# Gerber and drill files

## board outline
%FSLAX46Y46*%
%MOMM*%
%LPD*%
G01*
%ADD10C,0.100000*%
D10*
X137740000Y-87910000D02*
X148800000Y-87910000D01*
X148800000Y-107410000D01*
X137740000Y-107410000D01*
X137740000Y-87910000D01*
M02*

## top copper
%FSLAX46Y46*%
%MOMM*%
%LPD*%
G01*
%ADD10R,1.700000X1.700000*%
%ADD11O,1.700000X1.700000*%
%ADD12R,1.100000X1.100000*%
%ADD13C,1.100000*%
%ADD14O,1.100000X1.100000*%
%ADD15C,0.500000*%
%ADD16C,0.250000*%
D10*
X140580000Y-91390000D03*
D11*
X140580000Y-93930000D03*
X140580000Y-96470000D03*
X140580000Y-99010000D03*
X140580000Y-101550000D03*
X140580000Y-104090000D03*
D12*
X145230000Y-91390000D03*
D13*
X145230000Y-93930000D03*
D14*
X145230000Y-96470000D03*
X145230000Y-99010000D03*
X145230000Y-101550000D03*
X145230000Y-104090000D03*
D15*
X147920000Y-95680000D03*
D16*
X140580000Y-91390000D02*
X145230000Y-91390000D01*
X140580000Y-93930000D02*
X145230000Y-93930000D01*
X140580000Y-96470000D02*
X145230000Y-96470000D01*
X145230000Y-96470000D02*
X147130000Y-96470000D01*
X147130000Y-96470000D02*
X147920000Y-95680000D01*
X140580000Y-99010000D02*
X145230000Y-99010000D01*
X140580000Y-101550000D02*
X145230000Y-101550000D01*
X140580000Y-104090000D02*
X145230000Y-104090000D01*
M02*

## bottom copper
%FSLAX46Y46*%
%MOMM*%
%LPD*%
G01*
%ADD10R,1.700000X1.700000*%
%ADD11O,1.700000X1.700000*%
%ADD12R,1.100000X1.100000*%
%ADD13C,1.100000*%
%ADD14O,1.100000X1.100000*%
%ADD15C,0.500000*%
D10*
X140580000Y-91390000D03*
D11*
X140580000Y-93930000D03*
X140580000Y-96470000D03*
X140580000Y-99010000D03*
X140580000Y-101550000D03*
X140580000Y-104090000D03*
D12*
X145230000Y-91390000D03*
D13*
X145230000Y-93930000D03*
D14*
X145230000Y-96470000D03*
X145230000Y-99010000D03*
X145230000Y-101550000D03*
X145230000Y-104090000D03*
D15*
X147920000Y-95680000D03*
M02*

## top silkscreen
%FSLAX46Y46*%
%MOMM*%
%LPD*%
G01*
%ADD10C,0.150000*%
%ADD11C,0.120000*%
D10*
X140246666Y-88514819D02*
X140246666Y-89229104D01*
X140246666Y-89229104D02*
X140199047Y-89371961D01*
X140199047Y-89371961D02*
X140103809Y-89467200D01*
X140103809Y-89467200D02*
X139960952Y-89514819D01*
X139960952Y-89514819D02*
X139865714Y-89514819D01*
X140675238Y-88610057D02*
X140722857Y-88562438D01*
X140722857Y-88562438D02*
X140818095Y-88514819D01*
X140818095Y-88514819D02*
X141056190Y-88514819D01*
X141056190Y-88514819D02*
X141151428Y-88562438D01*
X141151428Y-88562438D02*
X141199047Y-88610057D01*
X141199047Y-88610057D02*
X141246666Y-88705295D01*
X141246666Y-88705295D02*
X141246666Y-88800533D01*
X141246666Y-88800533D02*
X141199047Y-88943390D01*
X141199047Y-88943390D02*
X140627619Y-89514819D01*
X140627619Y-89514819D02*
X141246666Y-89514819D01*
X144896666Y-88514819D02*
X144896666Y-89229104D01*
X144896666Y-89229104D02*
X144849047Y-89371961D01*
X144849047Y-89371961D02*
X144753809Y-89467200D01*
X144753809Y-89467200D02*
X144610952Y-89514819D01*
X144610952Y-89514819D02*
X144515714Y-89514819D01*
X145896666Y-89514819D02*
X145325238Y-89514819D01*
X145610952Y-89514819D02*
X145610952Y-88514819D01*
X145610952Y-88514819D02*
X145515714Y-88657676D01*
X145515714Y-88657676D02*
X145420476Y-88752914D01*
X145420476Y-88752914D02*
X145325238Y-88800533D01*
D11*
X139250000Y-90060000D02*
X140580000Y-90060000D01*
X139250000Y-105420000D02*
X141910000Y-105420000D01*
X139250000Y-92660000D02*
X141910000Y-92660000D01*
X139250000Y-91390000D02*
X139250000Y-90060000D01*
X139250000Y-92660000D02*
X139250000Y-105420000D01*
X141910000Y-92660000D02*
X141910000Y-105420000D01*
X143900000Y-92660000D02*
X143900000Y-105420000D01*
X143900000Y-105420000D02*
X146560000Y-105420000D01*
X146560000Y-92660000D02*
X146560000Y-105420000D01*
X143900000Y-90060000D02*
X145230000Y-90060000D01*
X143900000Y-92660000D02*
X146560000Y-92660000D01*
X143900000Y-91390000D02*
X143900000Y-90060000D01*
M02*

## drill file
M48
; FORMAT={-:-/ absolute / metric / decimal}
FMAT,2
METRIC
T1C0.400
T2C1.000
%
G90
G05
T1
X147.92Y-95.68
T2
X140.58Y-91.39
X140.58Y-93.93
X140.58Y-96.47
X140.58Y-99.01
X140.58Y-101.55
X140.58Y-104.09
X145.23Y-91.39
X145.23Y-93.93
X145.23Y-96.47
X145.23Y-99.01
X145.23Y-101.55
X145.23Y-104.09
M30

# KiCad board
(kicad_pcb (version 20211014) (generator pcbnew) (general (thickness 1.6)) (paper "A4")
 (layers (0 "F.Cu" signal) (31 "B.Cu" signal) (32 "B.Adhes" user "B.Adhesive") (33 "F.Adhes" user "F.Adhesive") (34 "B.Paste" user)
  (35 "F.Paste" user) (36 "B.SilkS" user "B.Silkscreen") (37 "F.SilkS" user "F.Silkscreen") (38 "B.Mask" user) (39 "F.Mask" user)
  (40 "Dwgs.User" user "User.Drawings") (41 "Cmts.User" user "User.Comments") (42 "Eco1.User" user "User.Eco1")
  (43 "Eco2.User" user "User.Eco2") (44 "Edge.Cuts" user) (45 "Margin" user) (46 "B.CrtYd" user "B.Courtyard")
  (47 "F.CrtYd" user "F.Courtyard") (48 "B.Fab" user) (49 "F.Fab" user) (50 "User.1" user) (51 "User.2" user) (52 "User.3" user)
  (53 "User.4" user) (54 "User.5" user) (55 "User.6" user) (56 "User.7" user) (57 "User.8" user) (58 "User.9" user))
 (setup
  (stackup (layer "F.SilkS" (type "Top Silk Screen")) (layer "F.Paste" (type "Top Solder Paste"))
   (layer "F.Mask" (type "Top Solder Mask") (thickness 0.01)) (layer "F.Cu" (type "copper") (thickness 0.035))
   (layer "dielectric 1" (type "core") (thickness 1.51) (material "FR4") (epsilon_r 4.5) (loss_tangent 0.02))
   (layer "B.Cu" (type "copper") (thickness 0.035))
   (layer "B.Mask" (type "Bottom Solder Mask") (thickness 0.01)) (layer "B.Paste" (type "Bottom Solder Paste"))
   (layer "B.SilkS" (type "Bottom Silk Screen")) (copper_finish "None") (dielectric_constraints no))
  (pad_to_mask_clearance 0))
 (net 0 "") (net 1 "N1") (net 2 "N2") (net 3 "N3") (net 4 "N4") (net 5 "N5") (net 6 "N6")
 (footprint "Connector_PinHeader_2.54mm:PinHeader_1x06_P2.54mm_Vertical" (layer "F.Cu") (at 140.58 91.39)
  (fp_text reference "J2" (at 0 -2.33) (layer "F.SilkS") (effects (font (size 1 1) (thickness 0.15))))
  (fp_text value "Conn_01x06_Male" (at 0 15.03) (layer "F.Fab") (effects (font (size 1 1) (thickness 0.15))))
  (fp_line (start -1.33 -1.33) (end 0 -1.33) (layer "F.SilkS") (width 0.12))
  (fp_line (start -1.33 14.03) (end 1.33 14.03) (layer "F.SilkS") (width 0.12))
  (fp_line (start -1.33 1.27) (end 1.33 1.27) (layer "F.SilkS") (width 0.12))
  (fp_line (start -1.33 0) (end -1.33 -1.33) (layer "F.SilkS") (width 0.12))
  (fp_line (start -1.33 1.27) (end -1.33 14.03) (layer "F.SilkS") (width 0.12))
  (fp_line (start 1.33 1.27) (end 1.33 14.03) (layer "F.SilkS") (width 0.12))
  (pad "1" thru_hole rect (at 0 0) (size 1.7 1.7) (drill 1) (layers *.Cu *.Mask) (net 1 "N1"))
  (pad "2" thru_hole oval (at 0 2.54) (size 1.7 1.7) (drill 1) (layers *.Cu *.Mask) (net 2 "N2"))
  (pad "3" thru_hole oval (at 0 5.08) (size 1.7 1.7) (drill 1) (layers *.Cu *.Mask) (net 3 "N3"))
  (pad "4" thru_hole oval (at 0 7.62) (size 1.7 1.7) (drill 1) (layers *.Cu *.Mask) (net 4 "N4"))
  (pad "5" thru_hole oval (at 0 10.16) (size 1.7 1.7) (drill 1) (layers *.Cu *.Mask) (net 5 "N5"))
  (pad "6" thru_hole oval (at 0 12.7) (size 1.7 1.7) (drill 1) (layers *.Cu *.Mask) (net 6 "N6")))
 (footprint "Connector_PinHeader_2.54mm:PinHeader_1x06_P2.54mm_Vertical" (layer "F.Cu") (at 145.23 91.39)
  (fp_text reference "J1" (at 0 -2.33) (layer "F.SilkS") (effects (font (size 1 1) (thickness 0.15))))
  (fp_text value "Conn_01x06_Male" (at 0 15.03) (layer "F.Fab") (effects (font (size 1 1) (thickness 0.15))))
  (fp_line (start -1.33 1.27) (end -1.33 14.03) (layer "F.SilkS") (width 0.12))
  (fp_line (start -1.33 14.03) (end 1.33 14.03) (layer "F.SilkS") (width 0.12))
  (fp_line (start 1.33 1.27) (end 1.33 14.03) (layer "F.SilkS") (width 0.12))
  (fp_line (start -1.33 -1.33) (end 0 -1.33) (layer "F.SilkS") (width 0.12))
  (fp_line (start -1.33 1.27) (end 1.33 1.27) (layer "F.SilkS") (width 0.12))
  (fp_line (start -1.33 0) (end -1.33 -1.33) (layer "F.SilkS") (width 0.12))
  (pad "1" thru_hole rect (at 0 0) (size 1.1 1.1) (drill 1) (layers *.Cu *.Mask) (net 1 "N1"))
  (pad "2" thru_hole circle (at 0 2.54) (size 1.1 1.1) (drill 1) (layers *.Cu *.Mask) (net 2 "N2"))
  (pad "3" thru_hole oval (at 0 5.08) (size 1.1 1.1) (drill 1) (layers *.Cu *.Mask) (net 3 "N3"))
  (pad "4" thru_hole oval (at 0 7.62) (size 1.1 1.1) (drill 1) (layers *.Cu *.Mask) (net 4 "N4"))
  (pad "5" thru_hole oval (at 0 10.16) (size 1.1 1.1) (drill 1) (layers *.Cu *.Mask) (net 5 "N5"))
  (pad "6" thru_hole oval (at 0 12.7) (size 1.1 1.1) (drill 1) (layers *.Cu *.Mask) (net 6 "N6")))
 (gr_rect (start 137.74 87.91) (end 148.8 107.41) (layer "Edge.Cuts") (width 0.1) (fill none))
 (segment (start 140.58 91.39) (end 145.23 91.39) (width 0.25) (layer "F.Cu") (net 1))
 (segment (start 140.58 93.93) (end 145.23 93.93) (width 0.25) (layer "F.Cu") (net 2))
 (segment (start 140.58 96.47) (end 145.23 96.47) (width 0.25) (layer "F.Cu") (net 3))
 (segment (start 145.23 96.47) (end 147.13 96.47) (width 0.25) (layer "F.Cu") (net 3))
 (segment (start 147.13 96.47) (end 147.92 95.68) (width 0.25) (layer "F.Cu") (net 3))
 (via (at 147.92 95.68) (size 0.5) (drill 0.4) (layers "F.Cu" "B.Cu") (free) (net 3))
 (segment (start 140.58 99.01) (end 145.23 99.01) (width 0.25) (layer "F.Cu") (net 4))
 (segment (start 140.58 101.55) (end 145.23 101.55) (width 0.25) (layer "F.Cu") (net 5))
 (segment (start 140.58 104.09) (end 145.23 104.09) (width 0.25) (layer "F.Cu") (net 6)))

